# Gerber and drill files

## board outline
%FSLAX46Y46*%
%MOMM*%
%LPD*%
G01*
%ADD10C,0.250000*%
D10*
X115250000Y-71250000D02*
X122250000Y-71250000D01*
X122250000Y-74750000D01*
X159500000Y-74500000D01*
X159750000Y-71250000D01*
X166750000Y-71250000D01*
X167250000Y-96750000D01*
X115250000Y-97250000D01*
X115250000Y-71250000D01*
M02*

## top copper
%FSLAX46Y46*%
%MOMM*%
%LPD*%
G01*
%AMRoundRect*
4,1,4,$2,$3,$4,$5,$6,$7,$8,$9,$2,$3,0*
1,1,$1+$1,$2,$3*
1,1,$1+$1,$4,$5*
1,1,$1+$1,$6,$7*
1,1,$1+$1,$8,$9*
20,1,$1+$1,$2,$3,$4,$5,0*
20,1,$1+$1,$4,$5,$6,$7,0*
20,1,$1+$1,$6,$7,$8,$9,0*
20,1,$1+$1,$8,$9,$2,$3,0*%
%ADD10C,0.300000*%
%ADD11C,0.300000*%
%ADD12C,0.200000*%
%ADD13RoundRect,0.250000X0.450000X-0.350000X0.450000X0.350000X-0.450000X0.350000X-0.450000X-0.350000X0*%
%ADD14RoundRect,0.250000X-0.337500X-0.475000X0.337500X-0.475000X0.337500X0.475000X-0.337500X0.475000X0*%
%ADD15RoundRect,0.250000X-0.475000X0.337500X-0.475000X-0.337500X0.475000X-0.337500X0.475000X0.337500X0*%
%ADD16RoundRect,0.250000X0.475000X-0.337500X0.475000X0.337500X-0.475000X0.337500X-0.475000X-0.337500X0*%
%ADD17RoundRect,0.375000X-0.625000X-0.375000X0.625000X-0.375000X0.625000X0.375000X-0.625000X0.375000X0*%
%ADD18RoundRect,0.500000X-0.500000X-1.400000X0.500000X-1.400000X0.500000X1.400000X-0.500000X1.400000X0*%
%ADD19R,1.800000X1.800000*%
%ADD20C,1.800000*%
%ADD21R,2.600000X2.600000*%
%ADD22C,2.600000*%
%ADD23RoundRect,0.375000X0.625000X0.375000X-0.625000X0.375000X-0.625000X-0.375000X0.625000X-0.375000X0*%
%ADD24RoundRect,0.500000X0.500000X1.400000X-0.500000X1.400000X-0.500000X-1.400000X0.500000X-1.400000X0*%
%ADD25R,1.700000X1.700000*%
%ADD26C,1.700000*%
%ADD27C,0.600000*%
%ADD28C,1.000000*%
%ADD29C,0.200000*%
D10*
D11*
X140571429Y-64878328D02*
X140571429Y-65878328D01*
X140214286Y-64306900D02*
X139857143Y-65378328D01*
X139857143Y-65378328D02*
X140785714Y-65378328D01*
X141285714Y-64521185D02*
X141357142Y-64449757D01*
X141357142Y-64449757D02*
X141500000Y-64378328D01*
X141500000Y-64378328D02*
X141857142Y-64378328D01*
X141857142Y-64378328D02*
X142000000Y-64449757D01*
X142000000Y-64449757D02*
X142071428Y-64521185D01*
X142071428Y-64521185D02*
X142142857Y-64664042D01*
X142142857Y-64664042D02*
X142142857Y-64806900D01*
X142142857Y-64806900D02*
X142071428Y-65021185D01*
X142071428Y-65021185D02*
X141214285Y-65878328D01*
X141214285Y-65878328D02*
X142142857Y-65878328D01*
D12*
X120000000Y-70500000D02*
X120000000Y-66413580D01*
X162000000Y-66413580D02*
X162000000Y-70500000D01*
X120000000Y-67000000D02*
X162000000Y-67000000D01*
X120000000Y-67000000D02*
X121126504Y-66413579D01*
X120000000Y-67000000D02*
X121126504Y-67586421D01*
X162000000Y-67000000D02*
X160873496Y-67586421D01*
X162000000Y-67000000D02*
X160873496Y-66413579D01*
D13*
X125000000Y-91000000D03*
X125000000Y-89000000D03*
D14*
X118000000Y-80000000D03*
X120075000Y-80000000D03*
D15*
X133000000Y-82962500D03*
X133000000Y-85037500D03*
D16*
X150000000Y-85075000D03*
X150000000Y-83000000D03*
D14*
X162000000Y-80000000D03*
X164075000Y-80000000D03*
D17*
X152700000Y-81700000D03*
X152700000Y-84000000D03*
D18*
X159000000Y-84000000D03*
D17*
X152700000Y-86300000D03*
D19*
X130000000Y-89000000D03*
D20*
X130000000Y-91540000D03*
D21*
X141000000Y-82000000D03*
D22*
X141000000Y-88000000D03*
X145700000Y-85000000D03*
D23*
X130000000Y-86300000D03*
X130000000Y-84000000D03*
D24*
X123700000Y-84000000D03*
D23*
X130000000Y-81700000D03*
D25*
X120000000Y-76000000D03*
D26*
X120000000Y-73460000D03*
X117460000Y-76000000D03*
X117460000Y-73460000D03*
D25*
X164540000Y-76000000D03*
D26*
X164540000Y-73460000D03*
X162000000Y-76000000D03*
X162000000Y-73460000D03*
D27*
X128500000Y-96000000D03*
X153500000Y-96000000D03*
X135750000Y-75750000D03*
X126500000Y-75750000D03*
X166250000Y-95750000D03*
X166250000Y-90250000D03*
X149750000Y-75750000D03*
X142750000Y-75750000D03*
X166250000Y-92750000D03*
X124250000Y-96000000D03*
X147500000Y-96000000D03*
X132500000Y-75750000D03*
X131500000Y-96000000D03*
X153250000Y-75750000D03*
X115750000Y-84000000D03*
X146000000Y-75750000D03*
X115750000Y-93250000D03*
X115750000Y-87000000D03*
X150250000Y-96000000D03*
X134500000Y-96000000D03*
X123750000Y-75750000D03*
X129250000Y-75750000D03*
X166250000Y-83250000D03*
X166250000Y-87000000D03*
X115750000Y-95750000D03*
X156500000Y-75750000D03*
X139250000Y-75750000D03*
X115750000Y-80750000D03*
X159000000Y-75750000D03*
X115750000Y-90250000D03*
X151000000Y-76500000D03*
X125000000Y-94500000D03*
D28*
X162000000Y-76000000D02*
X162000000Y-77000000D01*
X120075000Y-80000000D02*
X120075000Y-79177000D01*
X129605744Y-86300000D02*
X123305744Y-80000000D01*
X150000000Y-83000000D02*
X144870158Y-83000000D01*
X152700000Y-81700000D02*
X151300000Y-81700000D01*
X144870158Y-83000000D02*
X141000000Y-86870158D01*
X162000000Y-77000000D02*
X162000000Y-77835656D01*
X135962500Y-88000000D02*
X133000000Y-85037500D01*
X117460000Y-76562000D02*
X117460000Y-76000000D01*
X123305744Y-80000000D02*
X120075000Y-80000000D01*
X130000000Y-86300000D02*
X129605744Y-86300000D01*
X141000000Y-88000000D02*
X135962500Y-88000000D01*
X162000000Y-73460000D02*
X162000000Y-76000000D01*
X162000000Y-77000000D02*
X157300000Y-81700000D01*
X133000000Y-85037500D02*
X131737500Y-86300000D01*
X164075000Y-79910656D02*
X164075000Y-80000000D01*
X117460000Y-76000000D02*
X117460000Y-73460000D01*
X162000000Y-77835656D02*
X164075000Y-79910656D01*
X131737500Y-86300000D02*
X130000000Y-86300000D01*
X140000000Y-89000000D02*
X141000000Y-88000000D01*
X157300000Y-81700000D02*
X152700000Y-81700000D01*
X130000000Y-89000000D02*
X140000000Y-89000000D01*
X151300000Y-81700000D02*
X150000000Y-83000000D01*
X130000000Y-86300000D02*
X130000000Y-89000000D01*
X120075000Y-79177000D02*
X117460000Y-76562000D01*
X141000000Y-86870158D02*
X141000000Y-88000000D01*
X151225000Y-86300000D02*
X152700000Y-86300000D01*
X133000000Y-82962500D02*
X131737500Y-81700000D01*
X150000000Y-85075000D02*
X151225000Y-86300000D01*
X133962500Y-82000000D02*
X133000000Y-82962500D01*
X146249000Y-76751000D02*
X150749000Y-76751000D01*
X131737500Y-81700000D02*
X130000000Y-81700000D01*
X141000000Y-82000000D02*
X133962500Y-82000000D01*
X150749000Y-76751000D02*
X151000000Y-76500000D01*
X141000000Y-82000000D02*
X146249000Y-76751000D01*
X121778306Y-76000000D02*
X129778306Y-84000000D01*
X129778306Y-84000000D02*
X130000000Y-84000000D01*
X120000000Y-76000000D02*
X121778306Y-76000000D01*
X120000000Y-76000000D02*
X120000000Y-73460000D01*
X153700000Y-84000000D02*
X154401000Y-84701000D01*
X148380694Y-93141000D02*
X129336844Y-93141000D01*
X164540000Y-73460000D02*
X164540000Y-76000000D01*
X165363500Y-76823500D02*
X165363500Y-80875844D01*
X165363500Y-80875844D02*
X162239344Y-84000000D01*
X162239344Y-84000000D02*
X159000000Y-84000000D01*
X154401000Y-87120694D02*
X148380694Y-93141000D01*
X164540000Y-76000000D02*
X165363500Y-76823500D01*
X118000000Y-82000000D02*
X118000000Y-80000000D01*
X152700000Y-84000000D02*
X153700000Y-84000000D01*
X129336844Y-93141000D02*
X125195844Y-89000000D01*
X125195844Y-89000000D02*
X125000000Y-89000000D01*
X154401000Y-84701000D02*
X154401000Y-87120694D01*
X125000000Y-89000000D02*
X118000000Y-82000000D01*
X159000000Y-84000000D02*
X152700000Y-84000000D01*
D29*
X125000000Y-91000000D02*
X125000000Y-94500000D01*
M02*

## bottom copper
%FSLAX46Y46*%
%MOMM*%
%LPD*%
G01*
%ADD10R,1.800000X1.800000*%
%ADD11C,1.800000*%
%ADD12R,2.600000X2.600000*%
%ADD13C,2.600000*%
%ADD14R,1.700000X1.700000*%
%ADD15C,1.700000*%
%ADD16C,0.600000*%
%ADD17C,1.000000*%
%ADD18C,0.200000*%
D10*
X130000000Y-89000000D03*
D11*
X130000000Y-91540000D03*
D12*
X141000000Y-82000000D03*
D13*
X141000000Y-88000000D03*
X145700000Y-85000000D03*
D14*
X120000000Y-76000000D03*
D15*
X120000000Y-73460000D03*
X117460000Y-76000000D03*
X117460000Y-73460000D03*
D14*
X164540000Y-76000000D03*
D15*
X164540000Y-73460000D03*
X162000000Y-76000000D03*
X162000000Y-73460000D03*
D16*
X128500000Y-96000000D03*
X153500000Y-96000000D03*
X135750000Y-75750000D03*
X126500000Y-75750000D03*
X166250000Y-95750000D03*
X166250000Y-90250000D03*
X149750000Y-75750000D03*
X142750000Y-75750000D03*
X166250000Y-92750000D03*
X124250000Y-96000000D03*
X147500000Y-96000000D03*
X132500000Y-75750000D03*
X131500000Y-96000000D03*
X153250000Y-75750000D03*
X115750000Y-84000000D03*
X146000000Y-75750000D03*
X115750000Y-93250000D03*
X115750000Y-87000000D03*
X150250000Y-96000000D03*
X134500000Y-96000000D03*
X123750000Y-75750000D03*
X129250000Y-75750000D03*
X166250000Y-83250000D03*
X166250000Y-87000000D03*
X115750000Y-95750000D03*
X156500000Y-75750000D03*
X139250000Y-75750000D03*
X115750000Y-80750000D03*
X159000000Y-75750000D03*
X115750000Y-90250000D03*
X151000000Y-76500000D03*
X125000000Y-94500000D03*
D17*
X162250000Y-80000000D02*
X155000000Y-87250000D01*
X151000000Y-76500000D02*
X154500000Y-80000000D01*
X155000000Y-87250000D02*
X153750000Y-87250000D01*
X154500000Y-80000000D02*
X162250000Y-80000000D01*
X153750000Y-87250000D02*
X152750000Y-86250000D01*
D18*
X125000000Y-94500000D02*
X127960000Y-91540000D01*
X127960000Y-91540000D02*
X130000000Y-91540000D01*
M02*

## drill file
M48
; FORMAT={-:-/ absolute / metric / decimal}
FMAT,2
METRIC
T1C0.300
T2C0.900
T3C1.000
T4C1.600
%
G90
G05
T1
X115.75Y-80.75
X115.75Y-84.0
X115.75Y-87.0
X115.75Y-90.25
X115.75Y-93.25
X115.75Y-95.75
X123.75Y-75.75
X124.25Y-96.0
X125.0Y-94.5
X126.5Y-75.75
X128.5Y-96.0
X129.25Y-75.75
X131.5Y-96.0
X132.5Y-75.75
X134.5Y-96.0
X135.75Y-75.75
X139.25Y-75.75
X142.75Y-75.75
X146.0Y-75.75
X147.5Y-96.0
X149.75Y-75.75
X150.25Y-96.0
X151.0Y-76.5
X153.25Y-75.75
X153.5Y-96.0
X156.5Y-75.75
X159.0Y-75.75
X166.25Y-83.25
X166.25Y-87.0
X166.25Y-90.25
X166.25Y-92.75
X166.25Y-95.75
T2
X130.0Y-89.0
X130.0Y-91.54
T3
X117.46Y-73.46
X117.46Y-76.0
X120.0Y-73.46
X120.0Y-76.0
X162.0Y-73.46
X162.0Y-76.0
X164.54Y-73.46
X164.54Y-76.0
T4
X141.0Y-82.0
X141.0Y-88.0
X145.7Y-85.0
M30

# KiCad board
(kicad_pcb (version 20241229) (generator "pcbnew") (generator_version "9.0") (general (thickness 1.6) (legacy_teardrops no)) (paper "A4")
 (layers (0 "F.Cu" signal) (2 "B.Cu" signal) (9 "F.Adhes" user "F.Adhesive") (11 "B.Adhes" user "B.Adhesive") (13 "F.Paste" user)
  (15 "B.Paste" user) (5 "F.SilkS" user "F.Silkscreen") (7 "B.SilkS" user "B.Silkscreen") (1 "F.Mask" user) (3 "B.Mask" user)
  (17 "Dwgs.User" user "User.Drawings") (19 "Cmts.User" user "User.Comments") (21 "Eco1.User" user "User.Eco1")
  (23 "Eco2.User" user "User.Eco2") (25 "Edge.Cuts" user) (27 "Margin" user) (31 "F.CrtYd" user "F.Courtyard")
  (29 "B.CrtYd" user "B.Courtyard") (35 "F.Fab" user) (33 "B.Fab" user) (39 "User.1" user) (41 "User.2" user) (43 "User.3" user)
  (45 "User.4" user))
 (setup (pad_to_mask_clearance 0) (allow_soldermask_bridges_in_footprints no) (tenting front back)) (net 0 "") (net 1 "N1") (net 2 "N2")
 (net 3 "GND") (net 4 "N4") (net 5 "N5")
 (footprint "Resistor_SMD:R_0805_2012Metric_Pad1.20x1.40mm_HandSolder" (layer "F.Cu") (at 125 90 90)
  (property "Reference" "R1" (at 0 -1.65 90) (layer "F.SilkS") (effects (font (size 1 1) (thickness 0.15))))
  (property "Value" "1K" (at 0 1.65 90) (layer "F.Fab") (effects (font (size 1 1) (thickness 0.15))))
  (pad "1" smd roundrect (at -1 0 90) (size 1.2 1.4) (layers "F.Cu" "F.Mask" "F.Paste") (roundrect_rratio 0.208333) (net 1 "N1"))
  (pad "2" smd roundrect (at 1 0 90) (size 1.2 1.4) (layers "F.Cu" "F.Mask" "F.Paste") (roundrect_rratio 0.208333) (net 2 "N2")))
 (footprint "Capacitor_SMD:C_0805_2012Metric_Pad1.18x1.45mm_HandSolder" (layer "F.Cu") (at 119.0375 80)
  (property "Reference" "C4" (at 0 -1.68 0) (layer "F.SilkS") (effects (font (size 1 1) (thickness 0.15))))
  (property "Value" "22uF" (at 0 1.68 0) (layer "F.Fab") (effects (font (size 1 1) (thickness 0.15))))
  (pad "1" smd roundrect (at -1.0375 0) (size 1.175 1.45) (layers "F.Cu" "F.Mask" "F.Paste") (roundrect_rratio 0.212766) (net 2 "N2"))
  (pad "2" smd roundrect (at 1.0375 0) (size 1.175 1.45) (layers "F.Cu" "F.Mask" "F.Paste") (roundrect_rratio 0.212766) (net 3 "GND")))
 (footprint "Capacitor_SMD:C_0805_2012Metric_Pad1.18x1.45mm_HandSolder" (layer "F.Cu") (at 133 84 -90)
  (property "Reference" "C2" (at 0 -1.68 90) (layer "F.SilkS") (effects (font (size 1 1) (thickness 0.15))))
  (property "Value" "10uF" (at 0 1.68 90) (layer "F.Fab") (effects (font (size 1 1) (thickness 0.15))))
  (pad "1" smd roundrect (at -1.0375 0 270) (size 1.175 1.45) (layers "F.Cu" "F.Mask" "F.Paste") (roundrect_rratio 0.212766) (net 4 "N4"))
  (pad "2" smd roundrect (at 1.0375 0 270) (size 1.175 1.45) (layers "F.Cu" "F.Mask" "F.Paste") (roundrect_rratio 0.212766) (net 3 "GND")))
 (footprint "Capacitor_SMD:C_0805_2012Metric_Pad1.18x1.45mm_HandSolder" (layer "F.Cu") (at 150 84.0375 90)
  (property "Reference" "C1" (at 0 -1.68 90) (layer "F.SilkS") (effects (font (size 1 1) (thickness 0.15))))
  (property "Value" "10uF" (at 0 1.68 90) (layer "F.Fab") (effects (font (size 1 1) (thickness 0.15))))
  (pad "1" smd roundrect (at -1.0375 0 90) (size 1.175 1.45) (layers "F.Cu" "F.Mask" "F.Paste") (roundrect_rratio 0.212766) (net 4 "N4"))
  (pad "2" smd roundrect (at 1.0375 0 90) (size 1.175 1.45) (layers "F.Cu" "F.Mask" "F.Paste") (roundrect_rratio 0.212766) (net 3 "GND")))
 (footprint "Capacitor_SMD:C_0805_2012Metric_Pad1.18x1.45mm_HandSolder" (layer "F.Cu") (at 163.0375 80)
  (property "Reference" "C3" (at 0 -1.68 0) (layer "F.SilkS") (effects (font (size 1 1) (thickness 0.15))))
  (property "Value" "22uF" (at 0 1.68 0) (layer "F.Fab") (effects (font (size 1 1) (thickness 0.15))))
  (pad "1" smd roundrect (at -1.0375 0) (size 1.175 1.45) (layers "F.Cu" "F.Mask" "F.Paste") (roundrect_rratio 0.212766) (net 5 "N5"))
  (pad "2" smd roundrect (at 1.0375 0) (size 1.175 1.45) (layers "F.Cu" "F.Mask" "F.Paste") (roundrect_rratio 0.212766) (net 3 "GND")))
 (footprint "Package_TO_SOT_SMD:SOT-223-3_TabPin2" (layer "F.Cu") (at 155.85 84)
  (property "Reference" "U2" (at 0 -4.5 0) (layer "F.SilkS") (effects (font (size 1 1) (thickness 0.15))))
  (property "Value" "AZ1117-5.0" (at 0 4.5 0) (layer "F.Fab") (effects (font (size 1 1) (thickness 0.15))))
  (pad "1" smd roundrect (at -3.15 -2.3) (size 2 1.5) (layers "F.Cu" "F.Mask" "F.Paste") (roundrect_rratio 0.25) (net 3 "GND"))
  (pad "2" smd roundrect (at -3.15 0) (size 2 1.5) (layers "F.Cu" "F.Mask" "F.Paste") (roundrect_rratio 0.25) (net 2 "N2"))
  (pad "2" smd roundrect (at 3.15 0) (size 2 3.8) (layers "F.Cu" "F.Mask" "F.Paste") (roundrect_rratio 0.25) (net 2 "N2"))
  (pad "3" smd roundrect (at -3.15 2.3) (size 2 1.5) (layers "F.Cu" "F.Mask" "F.Paste") (roundrect_rratio 0.25) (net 4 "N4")))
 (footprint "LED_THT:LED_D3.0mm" (layer "F.Cu") (at 130 89 -90)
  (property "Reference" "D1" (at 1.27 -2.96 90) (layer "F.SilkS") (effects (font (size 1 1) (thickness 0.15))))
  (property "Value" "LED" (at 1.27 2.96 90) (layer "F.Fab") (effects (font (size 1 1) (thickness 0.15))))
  (pad "1" thru_hole rect (at 0 0 270) (size 1.8 1.8) (drill 0.9) (layers "*.Cu" "*.Mask") (remove_unused_layers no) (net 3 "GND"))
  (pad "2" thru_hole circle (at 2.54 0 270) (size 1.8 1.8) (drill 0.9) (layers "*.Cu" "*.Mask") (remove_unused_layers no) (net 1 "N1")))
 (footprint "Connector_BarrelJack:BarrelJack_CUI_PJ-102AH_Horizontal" (layer "F.Cu") (at 141 82)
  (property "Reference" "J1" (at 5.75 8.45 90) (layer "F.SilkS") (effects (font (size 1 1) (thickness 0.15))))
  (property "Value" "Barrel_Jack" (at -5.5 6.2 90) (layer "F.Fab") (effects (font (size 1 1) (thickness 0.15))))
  (pad "1" thru_hole rect (at 0 0) (size 2.6 2.6) (drill 1.6) (layers "*.Cu" "*.Mask") (remove_unused_layers no) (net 4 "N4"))
  (pad "2" thru_hole circle (at 0 6) (size 2.6 2.6) (drill 1.6) (layers "*.Cu" "*.Mask") (remove_unused_layers no) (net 3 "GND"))
  (pad "3" thru_hole circle (at 4.7 3) (size 2.6 2.6) (drill 1.6) (layers "*.Cu" "*.Mask") (remove_unused_layers no)))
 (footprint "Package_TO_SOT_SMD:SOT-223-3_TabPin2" (layer "F.Cu") (at 126.85 84 180)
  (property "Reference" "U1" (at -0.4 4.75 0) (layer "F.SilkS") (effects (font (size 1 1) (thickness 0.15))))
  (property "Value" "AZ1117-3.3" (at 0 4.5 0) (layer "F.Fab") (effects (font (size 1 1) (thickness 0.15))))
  (pad "1" smd roundrect (at -3.15 -2.3 180) (size 2 1.5) (layers "F.Cu" "F.Mask" "F.Paste") (roundrect_rratio 0.25) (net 3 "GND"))
  (pad "2" smd roundrect (at -3.15 0 180) (size 2 1.5) (layers "F.Cu" "F.Mask" "F.Paste") (roundrect_rratio 0.25) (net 5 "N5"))
  (pad "2" smd roundrect (at 3.15 0 180) (size 2 3.8) (layers "F.Cu" "F.Mask" "F.Paste") (roundrect_rratio 0.25) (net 5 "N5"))
  (pad "3" smd roundrect (at -3.15 2.3 180) (size 2 1.5) (layers "F.Cu" "F.Mask" "F.Paste") (roundrect_rratio 0.25) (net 4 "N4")))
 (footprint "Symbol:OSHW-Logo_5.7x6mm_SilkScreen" (layer "F.Cu") (at 119.5 93.25)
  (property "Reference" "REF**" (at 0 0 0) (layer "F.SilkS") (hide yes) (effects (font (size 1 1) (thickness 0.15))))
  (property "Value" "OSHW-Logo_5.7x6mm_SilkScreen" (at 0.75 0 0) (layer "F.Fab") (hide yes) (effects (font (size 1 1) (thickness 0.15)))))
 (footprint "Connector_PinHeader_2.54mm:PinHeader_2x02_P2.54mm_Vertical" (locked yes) (layer "B.Cu") (at 120 76 90)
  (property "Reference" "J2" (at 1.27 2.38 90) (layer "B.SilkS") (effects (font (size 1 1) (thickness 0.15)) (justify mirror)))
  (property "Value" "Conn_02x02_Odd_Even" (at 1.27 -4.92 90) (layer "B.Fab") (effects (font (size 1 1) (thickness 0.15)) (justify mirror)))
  (pad "1" thru_hole rect (at 0 0 90) (size 1.7 1.7) (drill 1) (layers "*.Cu" "*.Mask") (remove_unused_layers no) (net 5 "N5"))
  (pad "2" thru_hole circle (at 2.54 0 90) (size 1.7 1.7) (drill 1) (layers "*.Cu" "*.Mask") (remove_unused_layers no) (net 5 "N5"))
  (pad "3" thru_hole circle (at 0 -2.54 90) (size 1.7 1.7) (drill 1) (layers "*.Cu" "*.Mask") (remove_unused_layers no) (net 3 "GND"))
  (pad "4" thru_hole circle (at 2.54 -2.54 90) (size 1.7 1.7) (drill 1) (layers "*.Cu" "*.Mask") (remove_unused_layers no) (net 3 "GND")))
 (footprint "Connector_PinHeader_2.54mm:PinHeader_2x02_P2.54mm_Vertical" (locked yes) (layer "B.Cu") (at 164.54 76 90)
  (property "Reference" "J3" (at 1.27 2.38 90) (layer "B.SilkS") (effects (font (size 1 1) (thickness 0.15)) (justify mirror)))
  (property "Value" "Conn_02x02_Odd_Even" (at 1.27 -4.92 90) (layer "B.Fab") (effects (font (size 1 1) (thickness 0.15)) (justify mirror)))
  (pad "1" thru_hole rect (at 0 0 90) (size 1.7 1.7) (drill 1) (layers "*.Cu" "*.Mask") (remove_unused_layers no) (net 2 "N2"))
  (pad "2" thru_hole circle (at 2.54 0 90) (size 1.7 1.7) (drill 1) (layers "*.Cu" "*.Mask") (remove_unused_layers no) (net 2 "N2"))
  (pad "3" thru_hole circle (at 0 -2.54 90) (size 1.7 1.7) (drill 1) (layers "*.Cu" "*.Mask") (remove_unused_layers no) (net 3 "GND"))
  (pad "4" thru_hole circle (at 2.54 -2.54 90) (size 1.7 1.7) (drill 1) (layers "*.Cu" "*.Mask") (remove_unused_layers no) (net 3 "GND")))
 (gr_poly
  (pts (xy 115.25 71.25) (xy 122.25 71.25) (xy 122.25 74.75) (xy 159.5 74.5) (xy 159.75 71.25) (xy 166.75 71.25) (xy 167.25 96.75)
   (xy 115.25 97.25))
  (stroke (width 0.25) (type solid)) (fill no) (layer "Edge.Cuts"))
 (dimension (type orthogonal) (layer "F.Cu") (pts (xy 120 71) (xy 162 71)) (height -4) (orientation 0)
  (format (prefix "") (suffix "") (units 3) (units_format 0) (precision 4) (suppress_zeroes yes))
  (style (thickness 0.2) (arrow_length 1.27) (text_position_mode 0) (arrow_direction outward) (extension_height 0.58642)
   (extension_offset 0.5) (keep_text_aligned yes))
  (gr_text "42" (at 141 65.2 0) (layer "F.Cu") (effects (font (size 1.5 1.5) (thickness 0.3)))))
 (via (at 128.5 96) (size 0.6) (drill 0.3) (layers "F.Cu" "B.Cu") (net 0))
 (via (at 153.5 96) (size 0.6) (drill 0.3) (layers "F.Cu" "B.Cu") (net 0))
 (via (at 135.75 75.75) (size 0.6) (drill 0.3) (layers "F.Cu" "B.Cu") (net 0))
 (via (at 126.5 75.75) (size 0.6) (drill 0.3) (layers "F.Cu" "B.Cu") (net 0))
 (via (at 166.25 95.75) (size 0.6) (drill 0.3) (layers "F.Cu" "B.Cu") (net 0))
 (via (at 166.25 90.25) (size 0.6) (drill 0.3) (layers "F.Cu" "B.Cu") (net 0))
 (via (at 149.75 75.75) (size 0.6) (drill 0.3) (layers "F.Cu" "B.Cu") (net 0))
 (via (at 142.75 75.75) (size 0.6) (drill 0.3) (layers "F.Cu" "B.Cu") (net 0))
 (via (at 166.25 92.75) (size 0.6) (drill 0.3) (layers "F.Cu" "B.Cu") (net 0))
 (via (at 124.25 96) (size 0.6) (drill 0.3) (layers "F.Cu" "B.Cu") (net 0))
 (via (at 147.5 96) (size 0.6) (drill 0.3) (layers "F.Cu" "B.Cu") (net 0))
 (via (at 132.5 75.75) (size 0.6) (drill 0.3) (layers "F.Cu" "B.Cu") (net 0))
 (via (at 131.5 96) (size 0.6) (drill 0.3) (layers "F.Cu" "B.Cu") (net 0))
 (via (at 153.25 75.75) (size 0.6) (drill 0.3) (layers "F.Cu" "B.Cu") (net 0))
 (via (at 115.75 84) (size 0.6) (drill 0.3) (layers "F.Cu" "B.Cu") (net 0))
 (via (at 146 75.75) (size 0.6) (drill 0.3) (layers "F.Cu" "B.Cu") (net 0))
 (via (at 115.75 93.25) (size 0.6) (drill 0.3) (layers "F.Cu" "B.Cu") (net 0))
 (via (at 115.75 87) (size 0.6) (drill 0.3) (layers "F.Cu" "B.Cu") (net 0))
 (via (at 150.25 96) (size 0.6) (drill 0.3) (layers "F.Cu" "B.Cu") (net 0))
 (via (at 134.5 96) (size 0.6) (drill 0.3) (layers "F.Cu" "B.Cu") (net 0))
 (via (at 123.75 75.75) (size 0.6) (drill 0.3) (layers "F.Cu" "B.Cu") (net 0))
 (via (at 129.25 75.75) (size 0.6) (drill 0.3) (layers "F.Cu" "B.Cu") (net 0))
 (via (at 166.25 83.25) (size 0.6) (drill 0.3) (layers "F.Cu" "B.Cu") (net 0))
 (via (at 166.25 87) (size 0.6) (drill 0.3) (layers "F.Cu" "B.Cu") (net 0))
 (via (at 115.75 95.75) (size 0.6) (drill 0.3) (layers "F.Cu" "B.Cu") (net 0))
 (via (at 156.5 75.75) (size 0.6) (drill 0.3) (layers "F.Cu" "B.Cu") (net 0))
 (via (at 139.25 75.75) (size 0.6) (drill 0.3) (layers "F.Cu" "B.Cu") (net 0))
 (via (at 115.75 80.75) (size 0.6) (drill 0.3) (layers "F.Cu" "B.Cu") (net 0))
 (via (at 159 75.75) (size 0.6) (drill 0.3) (layers "F.Cu" "B.Cu") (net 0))
 (via (at 115.75 90.25) (size 0.6) (drill 0.3) (layers "F.Cu" "B.Cu") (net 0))
 (segment (start 162 76) (end 162 77) (width 1) (layer "F.Cu") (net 3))
 (segment (start 120.075 80) (end 120.075 79.177) (width 1) (layer "F.Cu") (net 3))
 (segment (start 129.605744 86.3) (end 123.305744 80) (width 1) (layer "F.Cu") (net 3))
 (segment (start 150 83) (end 144.870158 83) (width 1) (layer "F.Cu") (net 3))
 (segment (start 152.7 81.7) (end 151.3 81.7) (width 1) (layer "F.Cu") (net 3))
 (segment (start 144.870158 83) (end 141 86.870158) (width 1) (layer "F.Cu") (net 3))
 (segment (start 162 77) (end 162 77.835656) (width 1) (layer "F.Cu") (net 3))
 (segment (start 135.9625 88) (end 133 85.0375) (width 1) (layer "F.Cu") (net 3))
 (segment (start 117.46 76.562) (end 117.46 76) (width 1) (layer "F.Cu") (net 3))
 (segment (start 123.305744 80) (end 120.075 80) (width 1) (layer "F.Cu") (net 3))
 (segment (start 130 86.3) (end 129.605744 86.3) (width 1) (layer "F.Cu") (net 3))
 (segment (start 141 88) (end 135.9625 88) (width 1) (layer "F.Cu") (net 3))
 (segment (start 162 73.46) (end 162 76) (width 1) (layer "F.Cu") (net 3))
 (segment (start 162 77) (end 157.3 81.7) (width 1) (layer "F.Cu") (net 3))
 (segment (start 133 85.0375) (end 131.7375 86.3) (width 1) (layer "F.Cu") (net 3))
 (segment (start 164.075 79.910656) (end 164.075 80) (width 1) (layer "F.Cu") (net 3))
 (segment (start 117.46 76) (end 117.46 73.46) (width 1) (layer "F.Cu") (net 3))
 (segment (start 162 77.835656) (end 164.075 79.910656) (width 1) (layer "F.Cu") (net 3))
 (segment (start 131.7375 86.3) (end 130 86.3) (width 1) (layer "F.Cu") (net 3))
 (segment (start 140 89) (end 141 88) (width 1) (layer "F.Cu") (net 3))
 (segment (start 157.3 81.7) (end 152.7 81.7) (width 1) (layer "F.Cu") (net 3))
 (segment (start 130 89) (end 140 89) (width 1) (layer "F.Cu") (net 3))
 (segment (start 151.3 81.7) (end 150 83) (width 1) (layer "F.Cu") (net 3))
 (segment (start 130 86.3) (end 130 89) (width 1) (layer "F.Cu") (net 3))
 (segment (start 120.075 79.177) (end 117.46 76.562) (width 1) (layer "F.Cu") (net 3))
 (segment (start 141 86.870158) (end 141 88) (width 1) (layer "F.Cu") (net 3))
 (segment (start 151.225 86.3) (end 152.7 86.3) (width 1) (layer "F.Cu") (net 4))
 (segment (start 133 82.9625) (end 131.7375 81.7) (width 1) (layer "F.Cu") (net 4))
 (segment (start 150 85.075) (end 151.225 86.3) (width 1) (layer "F.Cu") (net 4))
 (segment (start 133.9625 82) (end 133 82.9625) (width 1) (layer "F.Cu") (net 4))
 (segment (start 146.249 76.751) (end 150.749 76.751) (width 1) (layer "F.Cu") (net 4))
 (segment (start 131.7375 81.7) (end 130 81.7) (width 1) (layer "F.Cu") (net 4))
 (segment (start 141 82) (end 133.9625 82) (width 1) (layer "F.Cu") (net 4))
 (segment (start 150.749 76.751) (end 151 76.5) (width 1) (layer "F.Cu") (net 4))
 (segment (start 141 82) (end 146.249 76.751) (width 1) (layer "F.Cu") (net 4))
 (via (at 151 76.5) (size 0.6) (drill 0.3) (layers "F.Cu" "B.Cu") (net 4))
 (segment (start 162.25 80) (end 155 87.25) (width 1) (layer "B.Cu") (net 4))
 (segment (start 151 76.5) (end 154.5 80) (width 1) (layer "B.Cu") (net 4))
 (segment (start 155 87.25) (end 153.75 87.25) (width 1) (layer "B.Cu") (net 4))
 (segment (start 154.5 80) (end 162.25 80) (width 1) (layer "B.Cu") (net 4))
 (segment (start 153.75 87.25) (end 152.75 86.25) (width 1) (layer "B.Cu") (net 4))
 (segment (start 121.778306 76) (end 129.778306 84) (width 1) (layer "F.Cu") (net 5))
 (segment (start 129.778306 84) (end 130 84) (width 1) (layer "F.Cu") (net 5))
 (segment (start 120 76) (end 121.778306 76) (width 1) (layer "F.Cu") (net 5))
 (segment (start 120 76) (end 120 73.46) (width 1) (layer "F.Cu") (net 5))
 (segment (start 153.7 84) (end 154.401 84.701) (width 1) (layer "F.Cu") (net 2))
 (segment (start 148.380694 93.141) (end 129.336844 93.141) (width 1) (layer "F.Cu") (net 2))
 (segment (start 164.54 73.46) (end 164.54 76) (width 1) (layer "F.Cu") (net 2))
 (segment (start 165.3635 76.8235) (end 165.3635 80.875844) (width 1) (layer "F.Cu") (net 2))
 (segment (start 165.3635 80.875844) (end 162.239344 84) (width 1) (layer "F.Cu") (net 2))
 (segment (start 162.239344 84) (end 159 84) (width 1) (layer "F.Cu") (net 2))
 (segment (start 154.401 87.120694) (end 148.380694 93.141) (width 1) (layer "F.Cu") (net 2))
 (segment (start 164.54 76) (end 165.3635 76.8235) (width 1) (layer "F.Cu") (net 2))
 (segment (start 118 82) (end 118 80) (width 1) (layer "F.Cu") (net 2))
 (segment (start 152.7 84) (end 153.7 84) (width 1) (layer "F.Cu") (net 2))
 (segment (start 129.336844 93.141) (end 125.195844 89) (width 1) (layer "F.Cu") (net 2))
 (segment (start 125.195844 89) (end 125 89) (width 1) (layer "F.Cu") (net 2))
 (segment (start 154.401 84.701) (end 154.401 87.120694) (width 1) (layer "F.Cu") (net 2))
 (segment (start 125 89) (end 118 82) (width 1) (layer "F.Cu") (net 2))
 (segment (start 159 84) (end 152.7 84) (width 1) (layer "F.Cu") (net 2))
 (segment (start 125 91) (end 125 94.5) (width 0.2) (layer "F.Cu") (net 1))
 (via (at 125 94.5) (size 0.6) (drill 0.3) (layers "F.Cu" "B.Cu") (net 1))
 (segment (start 125 94.5) (end 127.96 91.54) (width 0.2) (layer "B.Cu") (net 1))
 (segment (start 127.96 91.54) (end 130 91.54) (width 0.2) (layer "B.Cu") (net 1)))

